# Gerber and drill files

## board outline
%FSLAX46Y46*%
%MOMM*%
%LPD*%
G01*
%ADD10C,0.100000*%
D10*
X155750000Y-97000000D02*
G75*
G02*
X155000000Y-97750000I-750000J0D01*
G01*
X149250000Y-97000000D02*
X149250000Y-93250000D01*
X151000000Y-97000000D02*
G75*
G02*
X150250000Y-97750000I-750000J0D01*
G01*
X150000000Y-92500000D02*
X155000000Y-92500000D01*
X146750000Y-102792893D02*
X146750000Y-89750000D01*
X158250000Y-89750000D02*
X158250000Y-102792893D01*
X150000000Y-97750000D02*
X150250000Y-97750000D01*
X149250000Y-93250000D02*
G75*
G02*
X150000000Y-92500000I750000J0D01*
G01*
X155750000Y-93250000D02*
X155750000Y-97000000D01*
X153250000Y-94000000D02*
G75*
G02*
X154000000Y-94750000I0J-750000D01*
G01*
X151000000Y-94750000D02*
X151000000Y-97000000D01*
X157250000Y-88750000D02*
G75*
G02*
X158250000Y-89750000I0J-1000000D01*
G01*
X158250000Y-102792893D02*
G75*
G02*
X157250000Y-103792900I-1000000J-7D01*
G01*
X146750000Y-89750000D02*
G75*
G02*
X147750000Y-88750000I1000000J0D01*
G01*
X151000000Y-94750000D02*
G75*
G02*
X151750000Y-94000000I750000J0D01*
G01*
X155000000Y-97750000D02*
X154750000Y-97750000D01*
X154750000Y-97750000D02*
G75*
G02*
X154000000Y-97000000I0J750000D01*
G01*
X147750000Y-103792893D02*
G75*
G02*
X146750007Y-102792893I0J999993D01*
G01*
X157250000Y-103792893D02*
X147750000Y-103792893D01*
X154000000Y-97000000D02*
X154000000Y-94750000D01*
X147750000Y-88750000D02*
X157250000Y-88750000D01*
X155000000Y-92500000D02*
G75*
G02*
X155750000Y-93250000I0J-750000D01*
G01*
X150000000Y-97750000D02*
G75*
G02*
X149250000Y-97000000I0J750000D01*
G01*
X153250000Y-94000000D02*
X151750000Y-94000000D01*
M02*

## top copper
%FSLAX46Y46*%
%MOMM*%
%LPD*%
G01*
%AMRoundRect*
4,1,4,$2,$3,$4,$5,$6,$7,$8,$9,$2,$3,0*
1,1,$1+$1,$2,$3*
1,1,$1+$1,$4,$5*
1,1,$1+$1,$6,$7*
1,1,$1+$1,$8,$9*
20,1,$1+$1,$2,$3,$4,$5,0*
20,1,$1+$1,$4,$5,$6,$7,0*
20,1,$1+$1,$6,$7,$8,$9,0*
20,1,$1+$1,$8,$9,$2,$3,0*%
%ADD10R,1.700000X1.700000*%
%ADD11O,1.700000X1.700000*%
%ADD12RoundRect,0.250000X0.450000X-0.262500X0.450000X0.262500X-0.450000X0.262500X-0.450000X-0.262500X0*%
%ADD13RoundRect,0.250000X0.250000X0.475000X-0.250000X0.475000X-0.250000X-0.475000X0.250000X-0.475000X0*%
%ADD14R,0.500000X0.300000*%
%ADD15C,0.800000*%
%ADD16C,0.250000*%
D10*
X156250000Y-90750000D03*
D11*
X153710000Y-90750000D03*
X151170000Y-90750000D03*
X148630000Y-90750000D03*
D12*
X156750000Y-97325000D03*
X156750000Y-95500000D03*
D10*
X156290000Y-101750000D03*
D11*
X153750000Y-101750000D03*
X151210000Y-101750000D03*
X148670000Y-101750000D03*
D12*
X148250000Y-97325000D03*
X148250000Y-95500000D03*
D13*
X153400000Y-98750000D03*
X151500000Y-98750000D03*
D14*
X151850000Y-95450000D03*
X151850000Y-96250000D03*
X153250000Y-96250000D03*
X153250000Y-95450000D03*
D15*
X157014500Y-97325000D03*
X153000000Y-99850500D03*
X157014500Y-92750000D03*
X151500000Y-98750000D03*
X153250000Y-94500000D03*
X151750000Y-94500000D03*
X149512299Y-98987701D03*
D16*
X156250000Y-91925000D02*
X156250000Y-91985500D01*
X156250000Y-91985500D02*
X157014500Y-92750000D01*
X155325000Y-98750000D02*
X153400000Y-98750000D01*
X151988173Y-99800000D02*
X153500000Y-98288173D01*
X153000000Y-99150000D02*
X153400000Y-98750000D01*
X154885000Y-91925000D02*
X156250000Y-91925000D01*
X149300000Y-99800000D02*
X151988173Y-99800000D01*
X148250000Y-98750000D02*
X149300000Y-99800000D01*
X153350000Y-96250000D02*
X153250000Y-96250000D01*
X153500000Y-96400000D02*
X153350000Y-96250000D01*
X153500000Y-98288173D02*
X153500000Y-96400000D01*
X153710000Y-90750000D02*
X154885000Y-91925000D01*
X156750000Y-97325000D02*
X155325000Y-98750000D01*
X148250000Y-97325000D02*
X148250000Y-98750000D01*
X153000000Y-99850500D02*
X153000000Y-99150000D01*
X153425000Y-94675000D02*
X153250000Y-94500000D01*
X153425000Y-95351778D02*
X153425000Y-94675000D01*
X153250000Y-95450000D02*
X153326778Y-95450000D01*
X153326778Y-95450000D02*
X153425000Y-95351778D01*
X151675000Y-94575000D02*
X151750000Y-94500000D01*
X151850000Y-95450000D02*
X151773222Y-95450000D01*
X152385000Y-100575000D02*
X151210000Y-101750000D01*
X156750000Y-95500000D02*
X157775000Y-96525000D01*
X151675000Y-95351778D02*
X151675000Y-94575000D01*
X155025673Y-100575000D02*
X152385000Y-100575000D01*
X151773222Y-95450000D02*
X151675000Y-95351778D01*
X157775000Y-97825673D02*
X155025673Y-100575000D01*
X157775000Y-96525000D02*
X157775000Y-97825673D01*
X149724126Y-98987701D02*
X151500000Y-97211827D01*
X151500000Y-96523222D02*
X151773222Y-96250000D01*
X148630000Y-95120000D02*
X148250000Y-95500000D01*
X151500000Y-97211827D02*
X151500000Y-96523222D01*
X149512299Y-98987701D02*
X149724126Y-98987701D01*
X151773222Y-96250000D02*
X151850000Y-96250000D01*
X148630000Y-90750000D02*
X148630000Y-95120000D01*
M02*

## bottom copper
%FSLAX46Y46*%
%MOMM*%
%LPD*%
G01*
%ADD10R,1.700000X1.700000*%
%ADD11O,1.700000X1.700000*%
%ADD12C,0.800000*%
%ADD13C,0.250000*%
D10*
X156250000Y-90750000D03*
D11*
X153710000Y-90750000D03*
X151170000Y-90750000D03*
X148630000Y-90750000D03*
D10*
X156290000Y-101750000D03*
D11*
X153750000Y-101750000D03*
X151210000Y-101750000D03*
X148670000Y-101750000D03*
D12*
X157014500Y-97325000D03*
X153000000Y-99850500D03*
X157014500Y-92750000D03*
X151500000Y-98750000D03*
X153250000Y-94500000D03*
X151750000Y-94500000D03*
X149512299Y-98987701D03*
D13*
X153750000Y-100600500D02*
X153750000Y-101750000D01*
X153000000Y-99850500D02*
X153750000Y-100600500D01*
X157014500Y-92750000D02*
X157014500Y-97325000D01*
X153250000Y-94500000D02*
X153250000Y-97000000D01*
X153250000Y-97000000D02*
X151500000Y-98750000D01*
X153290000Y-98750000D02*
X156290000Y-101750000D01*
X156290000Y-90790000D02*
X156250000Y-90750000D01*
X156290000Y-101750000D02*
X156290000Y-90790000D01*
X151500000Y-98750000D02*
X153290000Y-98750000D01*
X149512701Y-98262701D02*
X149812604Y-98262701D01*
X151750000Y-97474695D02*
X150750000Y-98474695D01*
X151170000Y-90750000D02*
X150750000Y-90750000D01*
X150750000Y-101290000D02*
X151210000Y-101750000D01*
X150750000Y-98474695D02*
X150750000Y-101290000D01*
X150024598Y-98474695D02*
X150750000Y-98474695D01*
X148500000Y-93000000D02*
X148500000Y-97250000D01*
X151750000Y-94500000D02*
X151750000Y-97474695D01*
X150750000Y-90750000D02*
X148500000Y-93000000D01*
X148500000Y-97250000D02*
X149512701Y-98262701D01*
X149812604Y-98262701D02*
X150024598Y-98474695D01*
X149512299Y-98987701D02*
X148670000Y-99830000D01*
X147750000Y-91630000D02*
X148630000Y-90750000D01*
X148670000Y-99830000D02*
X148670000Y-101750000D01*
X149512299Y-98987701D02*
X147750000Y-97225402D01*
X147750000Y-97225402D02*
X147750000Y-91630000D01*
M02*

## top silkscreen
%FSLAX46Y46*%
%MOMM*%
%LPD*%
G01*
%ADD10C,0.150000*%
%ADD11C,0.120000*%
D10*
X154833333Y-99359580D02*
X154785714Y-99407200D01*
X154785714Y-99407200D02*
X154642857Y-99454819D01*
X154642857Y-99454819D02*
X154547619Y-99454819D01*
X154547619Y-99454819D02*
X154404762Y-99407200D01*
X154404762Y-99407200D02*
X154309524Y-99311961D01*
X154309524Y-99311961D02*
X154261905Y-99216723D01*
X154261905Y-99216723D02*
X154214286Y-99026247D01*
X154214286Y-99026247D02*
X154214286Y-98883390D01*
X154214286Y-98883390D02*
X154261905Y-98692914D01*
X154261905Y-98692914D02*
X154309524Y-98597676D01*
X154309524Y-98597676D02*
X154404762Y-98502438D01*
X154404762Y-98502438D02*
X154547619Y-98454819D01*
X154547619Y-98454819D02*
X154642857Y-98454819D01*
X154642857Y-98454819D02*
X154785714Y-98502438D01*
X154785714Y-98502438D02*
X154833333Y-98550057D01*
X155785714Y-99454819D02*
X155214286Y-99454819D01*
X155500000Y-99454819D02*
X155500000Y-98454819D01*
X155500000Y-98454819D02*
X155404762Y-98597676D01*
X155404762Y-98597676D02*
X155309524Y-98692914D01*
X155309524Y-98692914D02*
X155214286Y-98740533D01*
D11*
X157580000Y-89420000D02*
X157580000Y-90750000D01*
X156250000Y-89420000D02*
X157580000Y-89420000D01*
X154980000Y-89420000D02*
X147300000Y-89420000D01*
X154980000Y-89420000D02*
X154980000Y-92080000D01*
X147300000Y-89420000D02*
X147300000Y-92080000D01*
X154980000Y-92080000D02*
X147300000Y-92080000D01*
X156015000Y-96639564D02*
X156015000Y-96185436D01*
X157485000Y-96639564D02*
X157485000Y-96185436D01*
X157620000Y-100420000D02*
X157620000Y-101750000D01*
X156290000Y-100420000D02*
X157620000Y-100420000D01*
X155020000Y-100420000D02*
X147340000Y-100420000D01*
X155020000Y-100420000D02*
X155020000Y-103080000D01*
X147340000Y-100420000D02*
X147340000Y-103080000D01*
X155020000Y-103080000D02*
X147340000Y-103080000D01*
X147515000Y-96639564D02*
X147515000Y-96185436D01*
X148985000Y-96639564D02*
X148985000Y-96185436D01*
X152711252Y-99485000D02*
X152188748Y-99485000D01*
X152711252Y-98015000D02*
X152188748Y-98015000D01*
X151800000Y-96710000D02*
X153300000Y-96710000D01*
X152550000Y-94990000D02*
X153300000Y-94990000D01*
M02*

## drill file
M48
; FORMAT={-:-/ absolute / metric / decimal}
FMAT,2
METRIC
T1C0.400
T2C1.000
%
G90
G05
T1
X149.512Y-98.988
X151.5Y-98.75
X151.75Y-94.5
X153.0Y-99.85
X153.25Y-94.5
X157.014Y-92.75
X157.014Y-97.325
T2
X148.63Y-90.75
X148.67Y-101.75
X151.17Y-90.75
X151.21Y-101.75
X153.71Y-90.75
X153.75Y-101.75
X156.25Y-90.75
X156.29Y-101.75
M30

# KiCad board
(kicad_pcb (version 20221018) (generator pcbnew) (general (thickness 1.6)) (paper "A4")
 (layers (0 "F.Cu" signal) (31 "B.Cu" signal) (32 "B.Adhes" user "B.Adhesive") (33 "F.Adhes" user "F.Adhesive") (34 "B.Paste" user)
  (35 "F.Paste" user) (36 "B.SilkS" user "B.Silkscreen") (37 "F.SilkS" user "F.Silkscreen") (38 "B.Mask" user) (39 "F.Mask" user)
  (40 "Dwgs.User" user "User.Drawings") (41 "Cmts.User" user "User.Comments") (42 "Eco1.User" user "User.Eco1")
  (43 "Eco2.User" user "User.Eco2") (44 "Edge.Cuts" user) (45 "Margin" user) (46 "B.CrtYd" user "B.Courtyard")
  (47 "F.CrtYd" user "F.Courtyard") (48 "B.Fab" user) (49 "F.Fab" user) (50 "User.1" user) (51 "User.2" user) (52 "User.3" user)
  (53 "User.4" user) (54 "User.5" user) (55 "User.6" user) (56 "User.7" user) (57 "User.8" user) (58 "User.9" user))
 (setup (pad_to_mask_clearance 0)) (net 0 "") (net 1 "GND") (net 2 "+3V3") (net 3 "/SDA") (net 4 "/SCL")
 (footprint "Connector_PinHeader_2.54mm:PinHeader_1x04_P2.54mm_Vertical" (layer "F.Cu") (at 156.25 90.75 -90)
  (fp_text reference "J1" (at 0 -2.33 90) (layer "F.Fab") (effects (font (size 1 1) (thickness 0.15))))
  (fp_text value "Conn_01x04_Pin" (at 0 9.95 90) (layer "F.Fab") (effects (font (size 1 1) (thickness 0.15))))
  (fp_line (start -1.33 -1.33) (end 0 -1.33) (stroke (width 0.12) (type solid)) (layer "F.SilkS"))
  (fp_line (start -1.33 0) (end -1.33 -1.33) (stroke (width 0.12) (type solid)) (layer "F.SilkS"))
  (fp_line (start -1.33 1.27) (end -1.33 8.95) (stroke (width 0.12) (type solid)) (layer "F.SilkS"))
  (fp_line (start -1.33 1.27) (end 1.33 1.27) (stroke (width 0.12) (type solid)) (layer "F.SilkS"))
  (fp_line (start -1.33 8.95) (end 1.33 8.95) (stroke (width 0.12) (type solid)) (layer "F.SilkS"))
  (fp_line (start 1.33 1.27) (end 1.33 8.95) (stroke (width 0.12) (type solid)) (layer "F.SilkS"))
  (pad "1" thru_hole rect (at 0 0 270) (size 1.7 1.7) (drill 1) (layers "*.Cu" "*.Mask") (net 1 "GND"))
  (pad "2" thru_hole oval (at 0 2.54 270) (size 1.7 1.7) (drill 1) (layers "*.Cu" "*.Mask") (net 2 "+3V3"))
  (pad "3" thru_hole oval (at 0 5.08 270) (size 1.7 1.7) (drill 1) (layers "*.Cu" "*.Mask") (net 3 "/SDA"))
  (pad "4" thru_hole oval (at 0 7.62 270) (size 1.7 1.7) (drill 1) (layers "*.Cu" "*.Mask") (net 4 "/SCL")))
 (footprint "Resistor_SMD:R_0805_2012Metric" (layer "F.Cu") (at 156.75 96.4125 90)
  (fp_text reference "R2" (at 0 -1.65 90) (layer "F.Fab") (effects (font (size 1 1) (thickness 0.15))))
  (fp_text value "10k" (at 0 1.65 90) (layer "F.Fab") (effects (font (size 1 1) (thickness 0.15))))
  (fp_line (start -0.227064 -0.735) (end 0.227064 -0.735) (stroke (width 0.12) (type solid)) (layer "F.SilkS"))
  (fp_line (start -0.227064 0.735) (end 0.227064 0.735) (stroke (width 0.12) (type solid)) (layer "F.SilkS"))
  (pad "1" smd roundrect (at -0.9125 0 90) (size 1.025 1.4) (layers "F.Cu" "F.Paste" "F.Mask") (roundrect_rratio 0.243902) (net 2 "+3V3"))
  (pad "2" smd roundrect (at 0.9125 0 90) (size 1.025 1.4) (layers "F.Cu" "F.Paste" "F.Mask") (roundrect_rratio 0.243902) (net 3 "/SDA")))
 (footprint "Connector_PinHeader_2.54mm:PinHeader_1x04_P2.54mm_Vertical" (layer "F.Cu") (at 156.29 101.75 -90)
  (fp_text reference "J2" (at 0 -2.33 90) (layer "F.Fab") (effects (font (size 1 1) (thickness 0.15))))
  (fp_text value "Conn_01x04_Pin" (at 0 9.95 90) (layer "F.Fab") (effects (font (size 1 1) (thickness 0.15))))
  (fp_line (start -1.33 -1.33) (end 0 -1.33) (stroke (width 0.12) (type solid)) (layer "F.SilkS"))
  (fp_line (start -1.33 0) (end -1.33 -1.33) (stroke (width 0.12) (type solid)) (layer "F.SilkS"))
  (fp_line (start -1.33 1.27) (end -1.33 8.95) (stroke (width 0.12) (type solid)) (layer "F.SilkS"))
  (fp_line (start -1.33 1.27) (end 1.33 1.27) (stroke (width 0.12) (type solid)) (layer "F.SilkS"))
  (fp_line (start -1.33 8.95) (end 1.33 8.95) (stroke (width 0.12) (type solid)) (layer "F.SilkS"))
  (fp_line (start 1.33 1.27) (end 1.33 8.95) (stroke (width 0.12) (type solid)) (layer "F.SilkS"))
  (pad "1" thru_hole rect (at 0 0 270) (size 1.7 1.7) (drill 1) (layers "*.Cu" "*.Mask") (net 1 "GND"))
  (pad "2" thru_hole oval (at 0 2.54 270) (size 1.7 1.7) (drill 1) (layers "*.Cu" "*.Mask") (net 2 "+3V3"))
  (pad "3" thru_hole oval (at 0 5.08 270) (size 1.7 1.7) (drill 1) (layers "*.Cu" "*.Mask") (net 3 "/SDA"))
  (pad "4" thru_hole oval (at 0 7.62 270) (size 1.7 1.7) (drill 1) (layers "*.Cu" "*.Mask") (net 4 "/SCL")))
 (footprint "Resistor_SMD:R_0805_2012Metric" (layer "F.Cu") (at 148.25 96.4125 90)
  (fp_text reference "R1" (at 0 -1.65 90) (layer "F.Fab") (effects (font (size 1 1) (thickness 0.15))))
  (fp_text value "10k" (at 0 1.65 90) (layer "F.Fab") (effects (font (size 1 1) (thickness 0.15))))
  (fp_line (start -0.227064 -0.735) (end 0.227064 -0.735) (stroke (width 0.12) (type solid)) (layer "F.SilkS"))
  (fp_line (start -0.227064 0.735) (end 0.227064 0.735) (stroke (width 0.12) (type solid)) (layer "F.SilkS"))
  (pad "1" smd roundrect (at -0.9125 0 90) (size 1.025 1.4) (layers "F.Cu" "F.Paste" "F.Mask") (roundrect_rratio 0.243902) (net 2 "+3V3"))
  (pad "2" smd roundrect (at 0.9125 0 90) (size 1.025 1.4) (layers "F.Cu" "F.Paste" "F.Mask") (roundrect_rratio 0.243902) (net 4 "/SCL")))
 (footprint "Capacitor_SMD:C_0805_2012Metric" (layer "F.Cu") (at 152.45 98.75 180)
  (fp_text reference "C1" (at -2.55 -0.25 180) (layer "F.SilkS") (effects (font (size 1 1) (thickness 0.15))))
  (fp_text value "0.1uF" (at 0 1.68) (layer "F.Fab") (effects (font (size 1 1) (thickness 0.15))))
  (fp_line (start -0.261252 -0.735) (end 0.261252 -0.735) (stroke (width 0.12) (type solid)) (layer "F.SilkS"))
  (fp_line (start -0.261252 0.735) (end 0.261252 0.735) (stroke (width 0.12) (type solid)) (layer "F.SilkS"))
  (pad "1" smd roundrect (at -0.95 0 180) (size 1 1.45) (layers "F.Cu" "F.Paste" "F.Mask") (roundrect_rratio 0.25) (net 2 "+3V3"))
  (pad "2" smd roundrect (at 0.95 0 180) (size 1 1.45) (layers "F.Cu" "F.Paste" "F.Mask") (roundrect_rratio 0.25) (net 1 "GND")))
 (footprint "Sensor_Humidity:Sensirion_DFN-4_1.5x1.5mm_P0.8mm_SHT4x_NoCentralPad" (layer "F.Cu") (at 152.55 95.85)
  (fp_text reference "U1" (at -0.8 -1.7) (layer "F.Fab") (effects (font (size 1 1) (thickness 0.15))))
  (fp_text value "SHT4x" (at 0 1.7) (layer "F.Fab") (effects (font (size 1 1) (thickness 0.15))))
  (fp_line (start -0.75 0.86) (end 0.75 0.86) (stroke (width 0.12) (type solid)) (layer "F.SilkS"))
  (fp_line (start 0 -0.86) (end 0.75 -0.86) (stroke (width 0.12) (type solid)) (layer "F.SilkS"))
  (pad "1" smd rect (at -0.7 -0.4) (size 0.5 0.3) (layers "F.Cu" "F.Paste" "F.Mask") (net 3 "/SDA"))
  (pad "2" smd rect (at -0.7 0.4) (size 0.5 0.3) (layers "F.Cu" "F.Paste" "F.Mask") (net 4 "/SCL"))
  (pad "3" smd rect (at 0.7 0.4) (size 0.5 0.3) (layers "F.Cu" "F.Paste" "F.Mask") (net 2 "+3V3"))
  (pad "4" smd rect (at 0.7 -0.4) (size 0.5 0.3) (layers "F.Cu" "F.Paste" "F.Mask") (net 1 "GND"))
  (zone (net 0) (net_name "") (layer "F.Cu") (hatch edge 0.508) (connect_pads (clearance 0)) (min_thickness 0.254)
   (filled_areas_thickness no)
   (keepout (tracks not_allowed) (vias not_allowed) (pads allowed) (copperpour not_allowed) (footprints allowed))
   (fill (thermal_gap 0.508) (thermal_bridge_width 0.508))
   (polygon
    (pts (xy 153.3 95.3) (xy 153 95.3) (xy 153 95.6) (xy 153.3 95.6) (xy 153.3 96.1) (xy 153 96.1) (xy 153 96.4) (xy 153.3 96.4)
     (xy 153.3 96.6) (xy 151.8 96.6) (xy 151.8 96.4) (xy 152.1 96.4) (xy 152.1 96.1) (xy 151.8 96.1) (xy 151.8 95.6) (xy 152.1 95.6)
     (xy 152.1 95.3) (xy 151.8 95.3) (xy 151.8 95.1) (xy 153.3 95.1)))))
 (gr_arc (start 155.75 97) (mid 155.53033 97.53033) (end 155 97.75) (stroke (width 0.1) (type default)) (layer "Edge.Cuts"))
 (gr_line (start 149.25 97) (end 149.25 93.25) (stroke (width 0.1) (type default)) (layer "Edge.Cuts"))
 (gr_arc (start 151 97) (mid 150.78033 97.53033) (end 150.25 97.75) (stroke (width 0.1) (type default)) (layer "Edge.Cuts"))
 (gr_line (start 150 92.5) (end 155 92.5) (stroke (width 0.1) (type default)) (layer "Edge.Cuts"))
 (gr_line (start 146.75 102.792893) (end 146.75 89.75) (stroke (width 0.1) (type default)) (layer "Edge.Cuts"))
 (gr_line (start 158.25 89.75) (end 158.25 102.792893) (stroke (width 0.1) (type default)) (layer "Edge.Cuts"))
 (gr_line (start 150 97.75) (end 150.25 97.75) (stroke (width 0.1) (type default)) (layer "Edge.Cuts"))
 (gr_arc (start 149.25 93.25) (mid 149.46967 92.71967) (end 150 92.5) (stroke (width 0.1) (type default)) (layer "Edge.Cuts"))
 (gr_line (start 155.75 93.25) (end 155.75 97) (stroke (width 0.1) (type default)) (layer "Edge.Cuts"))
 (gr_arc (start 153.25 94) (mid 153.78033 94.21967) (end 154 94.75) (stroke (width 0.1) (type default)) (layer "Edge.Cuts"))
 (gr_line (start 151 94.75) (end 151 97) (stroke (width 0.1) (type default)) (layer "Edge.Cuts"))
 (gr_arc (start 157.25 88.75) (mid 157.957107 89.042893) (end 158.25 89.75) (stroke (width 0.1) (type default)) (layer "Edge.Cuts"))
 (gr_arc (start 158.25 102.792893) (mid 157.957107 103.5) (end 157.25 103.792893) (stroke (width 0.1) (type default)) (layer "Edge.Cuts"))
 (gr_arc (start 146.75 89.75) (mid 147.042893 89.042893) (end 147.75 88.75) (stroke (width 0.1) (type default)) (layer "Edge.Cuts"))
 (gr_arc (start 151 94.75) (mid 151.21967 94.21967) (end 151.75 94) (stroke (width 0.1) (type default)) (layer "Edge.Cuts"))
 (gr_line (start 155 97.75) (end 154.75 97.75) (stroke (width 0.1) (type default)) (layer "Edge.Cuts"))
 (gr_arc (start 154.75 97.75) (mid 154.21967 97.53033) (end 154 97) (stroke (width 0.1) (type default)) (layer "Edge.Cuts"))
 (gr_arc (start 147.75 103.792893) (mid 147.042893 103.5) (end 146.75 102.792893) (stroke (width 0.1) (type default)) (layer "Edge.Cuts"))
 (gr_line (start 157.25 103.792893) (end 147.75 103.792893) (stroke (width 0.1) (type default)) (layer "Edge.Cuts"))
 (gr_line (start 154 97) (end 154 94.75) (stroke (width 0.1) (type default)) (layer "Edge.Cuts"))
 (gr_line (start 147.75 88.75) (end 157.25 88.75) (stroke (width 0.1) (type default)) (layer "Edge.Cuts"))
 (gr_arc (start 155 92.5) (mid 155.53033 92.71967) (end 155.75 93.25) (stroke (width 0.1) (type default)) (layer "Edge.Cuts"))
 (gr_arc (start 150 97.75) (mid 149.46967 97.53033) (end 149.25 97) (stroke (width 0.1) (type default)) (layer "Edge.Cuts"))
 (gr_line (start 153.25 94) (end 151.75 94) (stroke (width 0.1) (type default)) (layer "Edge.Cuts"))
 (segment (start 156.25 91.925) (end 156.25 91.9855) (width 0.25) (layer "F.Cu") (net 2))
 (segment (start 156.25 91.9855) (end 157.0145 92.75) (width 0.25) (layer "F.Cu") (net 2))
 (segment (start 155.325 98.75) (end 153.4 98.75) (width 0.25) (layer "F.Cu") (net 2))
 (segment (start 151.988173 99.8) (end 153.5 98.288173) (width 0.25) (layer "F.Cu") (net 2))
 (segment (start 153 99.15) (end 153.4 98.75) (width 0.25) (layer "F.Cu") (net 2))
 (segment (start 154.885 91.925) (end 156.25 91.925) (width 0.25) (layer "F.Cu") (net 2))
 (segment (start 149.3 99.8) (end 151.988173 99.8) (width 0.25) (layer "F.Cu") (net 2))
 (segment (start 148.25 98.75) (end 149.3 99.8) (width 0.25) (layer "F.Cu") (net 2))
 (segment (start 153.35 96.25) (end 153.25 96.25) (width 0.25) (layer "F.Cu") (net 2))
 (segment (start 153.5 96.4) (end 153.35 96.25) (width 0.25) (layer "F.Cu") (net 2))
 (segment (start 153.5 98.288173) (end 153.5 96.4) (width 0.25) (layer "F.Cu") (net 2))
 (segment (start 153.71 90.75) (end 154.885 91.925) (width 0.25) (layer "F.Cu") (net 2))
 (segment (start 156.75 97.325) (end 155.325 98.75) (width 0.25) (layer "F.Cu") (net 2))
 (segment (start 148.25 97.325) (end 148.25 98.75) (width 0.25) (layer "F.Cu") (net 2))
 (segment (start 153 99.8505) (end 153 99.15) (width 0.25) (layer "F.Cu") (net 2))
 (via (at 157.0145 97.325) (size 0.8) (drill 0.4) (layers "F.Cu" "B.Cu") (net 2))
 (via (at 153 99.8505) (size 0.8) (drill 0.4) (layers "F.Cu" "B.Cu") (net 2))
 (via (at 157.0145 92.75) (size 0.8) (drill 0.4) (layers "F.Cu" "B.Cu") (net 2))
 (segment (start 153.75 100.6005) (end 153.75 101.75) (width 0.25) (layer "B.Cu") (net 2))
 (segment (start 153 99.8505) (end 153.75 100.6005) (width 0.25) (layer "B.Cu") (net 2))
 (segment (start 157.0145 92.75) (end 157.0145 97.325) (width 0.25) (layer "B.Cu") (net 2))
 (segment (start 153.425 94.675) (end 153.25 94.5) (width 0.25) (layer "F.Cu") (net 1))
 (segment (start 153.425 95.351778) (end 153.425 94.675) (width 0.25) (layer "F.Cu") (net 1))
 (segment (start 153.25 95.45) (end 153.326778 95.45) (width 0.25) (layer "F.Cu") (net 1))
 (segment (start 153.326778 95.45) (end 153.425 95.351778) (width 0.25) (layer "F.Cu") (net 1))
 (via (at 151.5 98.75) (size 0.8) (drill 0.4) (layers "F.Cu" "B.Cu") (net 1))
 (via (at 153.25 94.5) (size 0.8) (drill 0.4) (layers "F.Cu" "B.Cu") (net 1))
 (segment (start 153.25 94.5) (end 153.25 97) (width 0.25) (layer "B.Cu") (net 1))
 (segment (start 153.25 97) (end 151.5 98.75) (width 0.25) (layer "B.Cu") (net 1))
 (segment (start 153.29 98.75) (end 156.29 101.75) (width 0.25) (layer "B.Cu") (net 1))
 (segment (start 156.29 90.79) (end 156.25 90.75) (width 0.25) (layer "B.Cu") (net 1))
 (segment (start 156.29 101.75) (end 156.29 90.79) (width 0.25) (layer "B.Cu") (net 1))
 (segment (start 151.5 98.75) (end 153.29 98.75) (width 0.25) (layer "B.Cu") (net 1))
 (segment (start 151.675 94.575) (end 151.75 94.5) (width 0.25) (layer "F.Cu") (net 3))
 (segment (start 151.85 95.45) (end 151.773222 95.45) (width 0.25) (layer "F.Cu") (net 3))
 (segment (start 152.385 100.575) (end 151.21 101.75) (width 0.25) (layer "F.Cu") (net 3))
 (segment (start 156.75 95.5) (end 157.775 96.525) (width 0.25) (layer "F.Cu") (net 3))
 (segment (start 151.675 95.351778) (end 151.675 94.575) (width 0.25) (layer "F.Cu") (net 3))
 (segment (start 155.025673 100.575) (end 152.385 100.575) (width 0.25) (layer "F.Cu") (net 3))
 (segment (start 151.773222 95.45) (end 151.675 95.351778) (width 0.25) (layer "F.Cu") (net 3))
 (segment (start 157.775 97.825673) (end 155.025673 100.575) (width 0.25) (layer "F.Cu") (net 3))
 (segment (start 157.775 96.525) (end 157.775 97.825673) (width 0.25) (layer "F.Cu") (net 3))
 (via (at 151.75 94.5) (size 0.8) (drill 0.4) (layers "F.Cu" "B.Cu") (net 3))
 (segment (start 149.512701 98.262701) (end 149.812604 98.262701) (width 0.25) (layer "B.Cu") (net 3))
 (segment (start 151.75 97.474695) (end 150.75 98.474695) (width 0.25) (layer "B.Cu") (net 3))
 (segment (start 151.17 90.75) (end 150.75 90.75) (width 0.25) (layer "B.Cu") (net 3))
 (segment (start 150.75 101.29) (end 151.21 101.75) (width 0.25) (layer "B.Cu") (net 3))
 (segment (start 150.75 98.474695) (end 150.75 101.29) (width 0.25) (layer "B.Cu") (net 3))
 (segment (start 150.024598 98.474695) (end 150.75 98.474695) (width 0.25) (layer "B.Cu") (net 3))
 (segment (start 148.5 93) (end 148.5 97.25) (width 0.25) (layer "B.Cu") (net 3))
 (segment (start 151.75 94.5) (end 151.75 97.474695) (width 0.25) (layer "B.Cu") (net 3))
 (segment (start 150.75 90.75) (end 148.5 93) (width 0.25) (layer "B.Cu") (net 3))
 (segment (start 148.5 97.25) (end 149.512701 98.262701) (width 0.25) (layer "B.Cu") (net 3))
 (segment (start 149.812604 98.262701) (end 150.024598 98.474695) (width 0.25) (layer "B.Cu") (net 3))
 (segment (start 149.724126 98.987701) (end 151.5 97.211827) (width 0.25) (layer "F.Cu") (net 4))
 (segment (start 151.5 96.523222) (end 151.773222 96.25) (width 0.25) (layer "F.Cu") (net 4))
 (segment (start 148.63 95.12) (end 148.25 95.5) (width 0.25) (layer "F.Cu") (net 4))
 (segment (start 151.5 97.211827) (end 151.5 96.523222) (width 0.25) (layer "F.Cu") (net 4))
 (segment (start 149.512299 98.987701) (end 149.724126 98.987701) (width 0.25) (layer "F.Cu") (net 4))
 (segment (start 151.773222 96.25) (end 151.85 96.25) (width 0.25) (layer "F.Cu") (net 4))
 (segment (start 148.63 90.75) (end 148.63 95.12) (width 0.25) (layer "F.Cu") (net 4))
 (via (at 149.512299 98.987701) (size 0.8) (drill 0.4) (layers "F.Cu" "B.Cu") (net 4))
 (segment (start 149.512299 98.987701) (end 148.67 99.83) (width 0.25) (layer "B.Cu") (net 4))
 (segment (start 147.75 91.63) (end 148.63 90.75) (width 0.25) (layer "B.Cu") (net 4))
 (segment (start 148.67 99.83) (end 148.67 101.75) (width 0.25) (layer "B.Cu") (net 4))
 (segment (start 149.512299 98.987701) (end 147.75 97.225402) (width 0.25) (layer "B.Cu") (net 4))
 (segment (start 147.75 97.225402) (end 147.75 91.63) (width 0.25) (layer "B.Cu") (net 4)))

